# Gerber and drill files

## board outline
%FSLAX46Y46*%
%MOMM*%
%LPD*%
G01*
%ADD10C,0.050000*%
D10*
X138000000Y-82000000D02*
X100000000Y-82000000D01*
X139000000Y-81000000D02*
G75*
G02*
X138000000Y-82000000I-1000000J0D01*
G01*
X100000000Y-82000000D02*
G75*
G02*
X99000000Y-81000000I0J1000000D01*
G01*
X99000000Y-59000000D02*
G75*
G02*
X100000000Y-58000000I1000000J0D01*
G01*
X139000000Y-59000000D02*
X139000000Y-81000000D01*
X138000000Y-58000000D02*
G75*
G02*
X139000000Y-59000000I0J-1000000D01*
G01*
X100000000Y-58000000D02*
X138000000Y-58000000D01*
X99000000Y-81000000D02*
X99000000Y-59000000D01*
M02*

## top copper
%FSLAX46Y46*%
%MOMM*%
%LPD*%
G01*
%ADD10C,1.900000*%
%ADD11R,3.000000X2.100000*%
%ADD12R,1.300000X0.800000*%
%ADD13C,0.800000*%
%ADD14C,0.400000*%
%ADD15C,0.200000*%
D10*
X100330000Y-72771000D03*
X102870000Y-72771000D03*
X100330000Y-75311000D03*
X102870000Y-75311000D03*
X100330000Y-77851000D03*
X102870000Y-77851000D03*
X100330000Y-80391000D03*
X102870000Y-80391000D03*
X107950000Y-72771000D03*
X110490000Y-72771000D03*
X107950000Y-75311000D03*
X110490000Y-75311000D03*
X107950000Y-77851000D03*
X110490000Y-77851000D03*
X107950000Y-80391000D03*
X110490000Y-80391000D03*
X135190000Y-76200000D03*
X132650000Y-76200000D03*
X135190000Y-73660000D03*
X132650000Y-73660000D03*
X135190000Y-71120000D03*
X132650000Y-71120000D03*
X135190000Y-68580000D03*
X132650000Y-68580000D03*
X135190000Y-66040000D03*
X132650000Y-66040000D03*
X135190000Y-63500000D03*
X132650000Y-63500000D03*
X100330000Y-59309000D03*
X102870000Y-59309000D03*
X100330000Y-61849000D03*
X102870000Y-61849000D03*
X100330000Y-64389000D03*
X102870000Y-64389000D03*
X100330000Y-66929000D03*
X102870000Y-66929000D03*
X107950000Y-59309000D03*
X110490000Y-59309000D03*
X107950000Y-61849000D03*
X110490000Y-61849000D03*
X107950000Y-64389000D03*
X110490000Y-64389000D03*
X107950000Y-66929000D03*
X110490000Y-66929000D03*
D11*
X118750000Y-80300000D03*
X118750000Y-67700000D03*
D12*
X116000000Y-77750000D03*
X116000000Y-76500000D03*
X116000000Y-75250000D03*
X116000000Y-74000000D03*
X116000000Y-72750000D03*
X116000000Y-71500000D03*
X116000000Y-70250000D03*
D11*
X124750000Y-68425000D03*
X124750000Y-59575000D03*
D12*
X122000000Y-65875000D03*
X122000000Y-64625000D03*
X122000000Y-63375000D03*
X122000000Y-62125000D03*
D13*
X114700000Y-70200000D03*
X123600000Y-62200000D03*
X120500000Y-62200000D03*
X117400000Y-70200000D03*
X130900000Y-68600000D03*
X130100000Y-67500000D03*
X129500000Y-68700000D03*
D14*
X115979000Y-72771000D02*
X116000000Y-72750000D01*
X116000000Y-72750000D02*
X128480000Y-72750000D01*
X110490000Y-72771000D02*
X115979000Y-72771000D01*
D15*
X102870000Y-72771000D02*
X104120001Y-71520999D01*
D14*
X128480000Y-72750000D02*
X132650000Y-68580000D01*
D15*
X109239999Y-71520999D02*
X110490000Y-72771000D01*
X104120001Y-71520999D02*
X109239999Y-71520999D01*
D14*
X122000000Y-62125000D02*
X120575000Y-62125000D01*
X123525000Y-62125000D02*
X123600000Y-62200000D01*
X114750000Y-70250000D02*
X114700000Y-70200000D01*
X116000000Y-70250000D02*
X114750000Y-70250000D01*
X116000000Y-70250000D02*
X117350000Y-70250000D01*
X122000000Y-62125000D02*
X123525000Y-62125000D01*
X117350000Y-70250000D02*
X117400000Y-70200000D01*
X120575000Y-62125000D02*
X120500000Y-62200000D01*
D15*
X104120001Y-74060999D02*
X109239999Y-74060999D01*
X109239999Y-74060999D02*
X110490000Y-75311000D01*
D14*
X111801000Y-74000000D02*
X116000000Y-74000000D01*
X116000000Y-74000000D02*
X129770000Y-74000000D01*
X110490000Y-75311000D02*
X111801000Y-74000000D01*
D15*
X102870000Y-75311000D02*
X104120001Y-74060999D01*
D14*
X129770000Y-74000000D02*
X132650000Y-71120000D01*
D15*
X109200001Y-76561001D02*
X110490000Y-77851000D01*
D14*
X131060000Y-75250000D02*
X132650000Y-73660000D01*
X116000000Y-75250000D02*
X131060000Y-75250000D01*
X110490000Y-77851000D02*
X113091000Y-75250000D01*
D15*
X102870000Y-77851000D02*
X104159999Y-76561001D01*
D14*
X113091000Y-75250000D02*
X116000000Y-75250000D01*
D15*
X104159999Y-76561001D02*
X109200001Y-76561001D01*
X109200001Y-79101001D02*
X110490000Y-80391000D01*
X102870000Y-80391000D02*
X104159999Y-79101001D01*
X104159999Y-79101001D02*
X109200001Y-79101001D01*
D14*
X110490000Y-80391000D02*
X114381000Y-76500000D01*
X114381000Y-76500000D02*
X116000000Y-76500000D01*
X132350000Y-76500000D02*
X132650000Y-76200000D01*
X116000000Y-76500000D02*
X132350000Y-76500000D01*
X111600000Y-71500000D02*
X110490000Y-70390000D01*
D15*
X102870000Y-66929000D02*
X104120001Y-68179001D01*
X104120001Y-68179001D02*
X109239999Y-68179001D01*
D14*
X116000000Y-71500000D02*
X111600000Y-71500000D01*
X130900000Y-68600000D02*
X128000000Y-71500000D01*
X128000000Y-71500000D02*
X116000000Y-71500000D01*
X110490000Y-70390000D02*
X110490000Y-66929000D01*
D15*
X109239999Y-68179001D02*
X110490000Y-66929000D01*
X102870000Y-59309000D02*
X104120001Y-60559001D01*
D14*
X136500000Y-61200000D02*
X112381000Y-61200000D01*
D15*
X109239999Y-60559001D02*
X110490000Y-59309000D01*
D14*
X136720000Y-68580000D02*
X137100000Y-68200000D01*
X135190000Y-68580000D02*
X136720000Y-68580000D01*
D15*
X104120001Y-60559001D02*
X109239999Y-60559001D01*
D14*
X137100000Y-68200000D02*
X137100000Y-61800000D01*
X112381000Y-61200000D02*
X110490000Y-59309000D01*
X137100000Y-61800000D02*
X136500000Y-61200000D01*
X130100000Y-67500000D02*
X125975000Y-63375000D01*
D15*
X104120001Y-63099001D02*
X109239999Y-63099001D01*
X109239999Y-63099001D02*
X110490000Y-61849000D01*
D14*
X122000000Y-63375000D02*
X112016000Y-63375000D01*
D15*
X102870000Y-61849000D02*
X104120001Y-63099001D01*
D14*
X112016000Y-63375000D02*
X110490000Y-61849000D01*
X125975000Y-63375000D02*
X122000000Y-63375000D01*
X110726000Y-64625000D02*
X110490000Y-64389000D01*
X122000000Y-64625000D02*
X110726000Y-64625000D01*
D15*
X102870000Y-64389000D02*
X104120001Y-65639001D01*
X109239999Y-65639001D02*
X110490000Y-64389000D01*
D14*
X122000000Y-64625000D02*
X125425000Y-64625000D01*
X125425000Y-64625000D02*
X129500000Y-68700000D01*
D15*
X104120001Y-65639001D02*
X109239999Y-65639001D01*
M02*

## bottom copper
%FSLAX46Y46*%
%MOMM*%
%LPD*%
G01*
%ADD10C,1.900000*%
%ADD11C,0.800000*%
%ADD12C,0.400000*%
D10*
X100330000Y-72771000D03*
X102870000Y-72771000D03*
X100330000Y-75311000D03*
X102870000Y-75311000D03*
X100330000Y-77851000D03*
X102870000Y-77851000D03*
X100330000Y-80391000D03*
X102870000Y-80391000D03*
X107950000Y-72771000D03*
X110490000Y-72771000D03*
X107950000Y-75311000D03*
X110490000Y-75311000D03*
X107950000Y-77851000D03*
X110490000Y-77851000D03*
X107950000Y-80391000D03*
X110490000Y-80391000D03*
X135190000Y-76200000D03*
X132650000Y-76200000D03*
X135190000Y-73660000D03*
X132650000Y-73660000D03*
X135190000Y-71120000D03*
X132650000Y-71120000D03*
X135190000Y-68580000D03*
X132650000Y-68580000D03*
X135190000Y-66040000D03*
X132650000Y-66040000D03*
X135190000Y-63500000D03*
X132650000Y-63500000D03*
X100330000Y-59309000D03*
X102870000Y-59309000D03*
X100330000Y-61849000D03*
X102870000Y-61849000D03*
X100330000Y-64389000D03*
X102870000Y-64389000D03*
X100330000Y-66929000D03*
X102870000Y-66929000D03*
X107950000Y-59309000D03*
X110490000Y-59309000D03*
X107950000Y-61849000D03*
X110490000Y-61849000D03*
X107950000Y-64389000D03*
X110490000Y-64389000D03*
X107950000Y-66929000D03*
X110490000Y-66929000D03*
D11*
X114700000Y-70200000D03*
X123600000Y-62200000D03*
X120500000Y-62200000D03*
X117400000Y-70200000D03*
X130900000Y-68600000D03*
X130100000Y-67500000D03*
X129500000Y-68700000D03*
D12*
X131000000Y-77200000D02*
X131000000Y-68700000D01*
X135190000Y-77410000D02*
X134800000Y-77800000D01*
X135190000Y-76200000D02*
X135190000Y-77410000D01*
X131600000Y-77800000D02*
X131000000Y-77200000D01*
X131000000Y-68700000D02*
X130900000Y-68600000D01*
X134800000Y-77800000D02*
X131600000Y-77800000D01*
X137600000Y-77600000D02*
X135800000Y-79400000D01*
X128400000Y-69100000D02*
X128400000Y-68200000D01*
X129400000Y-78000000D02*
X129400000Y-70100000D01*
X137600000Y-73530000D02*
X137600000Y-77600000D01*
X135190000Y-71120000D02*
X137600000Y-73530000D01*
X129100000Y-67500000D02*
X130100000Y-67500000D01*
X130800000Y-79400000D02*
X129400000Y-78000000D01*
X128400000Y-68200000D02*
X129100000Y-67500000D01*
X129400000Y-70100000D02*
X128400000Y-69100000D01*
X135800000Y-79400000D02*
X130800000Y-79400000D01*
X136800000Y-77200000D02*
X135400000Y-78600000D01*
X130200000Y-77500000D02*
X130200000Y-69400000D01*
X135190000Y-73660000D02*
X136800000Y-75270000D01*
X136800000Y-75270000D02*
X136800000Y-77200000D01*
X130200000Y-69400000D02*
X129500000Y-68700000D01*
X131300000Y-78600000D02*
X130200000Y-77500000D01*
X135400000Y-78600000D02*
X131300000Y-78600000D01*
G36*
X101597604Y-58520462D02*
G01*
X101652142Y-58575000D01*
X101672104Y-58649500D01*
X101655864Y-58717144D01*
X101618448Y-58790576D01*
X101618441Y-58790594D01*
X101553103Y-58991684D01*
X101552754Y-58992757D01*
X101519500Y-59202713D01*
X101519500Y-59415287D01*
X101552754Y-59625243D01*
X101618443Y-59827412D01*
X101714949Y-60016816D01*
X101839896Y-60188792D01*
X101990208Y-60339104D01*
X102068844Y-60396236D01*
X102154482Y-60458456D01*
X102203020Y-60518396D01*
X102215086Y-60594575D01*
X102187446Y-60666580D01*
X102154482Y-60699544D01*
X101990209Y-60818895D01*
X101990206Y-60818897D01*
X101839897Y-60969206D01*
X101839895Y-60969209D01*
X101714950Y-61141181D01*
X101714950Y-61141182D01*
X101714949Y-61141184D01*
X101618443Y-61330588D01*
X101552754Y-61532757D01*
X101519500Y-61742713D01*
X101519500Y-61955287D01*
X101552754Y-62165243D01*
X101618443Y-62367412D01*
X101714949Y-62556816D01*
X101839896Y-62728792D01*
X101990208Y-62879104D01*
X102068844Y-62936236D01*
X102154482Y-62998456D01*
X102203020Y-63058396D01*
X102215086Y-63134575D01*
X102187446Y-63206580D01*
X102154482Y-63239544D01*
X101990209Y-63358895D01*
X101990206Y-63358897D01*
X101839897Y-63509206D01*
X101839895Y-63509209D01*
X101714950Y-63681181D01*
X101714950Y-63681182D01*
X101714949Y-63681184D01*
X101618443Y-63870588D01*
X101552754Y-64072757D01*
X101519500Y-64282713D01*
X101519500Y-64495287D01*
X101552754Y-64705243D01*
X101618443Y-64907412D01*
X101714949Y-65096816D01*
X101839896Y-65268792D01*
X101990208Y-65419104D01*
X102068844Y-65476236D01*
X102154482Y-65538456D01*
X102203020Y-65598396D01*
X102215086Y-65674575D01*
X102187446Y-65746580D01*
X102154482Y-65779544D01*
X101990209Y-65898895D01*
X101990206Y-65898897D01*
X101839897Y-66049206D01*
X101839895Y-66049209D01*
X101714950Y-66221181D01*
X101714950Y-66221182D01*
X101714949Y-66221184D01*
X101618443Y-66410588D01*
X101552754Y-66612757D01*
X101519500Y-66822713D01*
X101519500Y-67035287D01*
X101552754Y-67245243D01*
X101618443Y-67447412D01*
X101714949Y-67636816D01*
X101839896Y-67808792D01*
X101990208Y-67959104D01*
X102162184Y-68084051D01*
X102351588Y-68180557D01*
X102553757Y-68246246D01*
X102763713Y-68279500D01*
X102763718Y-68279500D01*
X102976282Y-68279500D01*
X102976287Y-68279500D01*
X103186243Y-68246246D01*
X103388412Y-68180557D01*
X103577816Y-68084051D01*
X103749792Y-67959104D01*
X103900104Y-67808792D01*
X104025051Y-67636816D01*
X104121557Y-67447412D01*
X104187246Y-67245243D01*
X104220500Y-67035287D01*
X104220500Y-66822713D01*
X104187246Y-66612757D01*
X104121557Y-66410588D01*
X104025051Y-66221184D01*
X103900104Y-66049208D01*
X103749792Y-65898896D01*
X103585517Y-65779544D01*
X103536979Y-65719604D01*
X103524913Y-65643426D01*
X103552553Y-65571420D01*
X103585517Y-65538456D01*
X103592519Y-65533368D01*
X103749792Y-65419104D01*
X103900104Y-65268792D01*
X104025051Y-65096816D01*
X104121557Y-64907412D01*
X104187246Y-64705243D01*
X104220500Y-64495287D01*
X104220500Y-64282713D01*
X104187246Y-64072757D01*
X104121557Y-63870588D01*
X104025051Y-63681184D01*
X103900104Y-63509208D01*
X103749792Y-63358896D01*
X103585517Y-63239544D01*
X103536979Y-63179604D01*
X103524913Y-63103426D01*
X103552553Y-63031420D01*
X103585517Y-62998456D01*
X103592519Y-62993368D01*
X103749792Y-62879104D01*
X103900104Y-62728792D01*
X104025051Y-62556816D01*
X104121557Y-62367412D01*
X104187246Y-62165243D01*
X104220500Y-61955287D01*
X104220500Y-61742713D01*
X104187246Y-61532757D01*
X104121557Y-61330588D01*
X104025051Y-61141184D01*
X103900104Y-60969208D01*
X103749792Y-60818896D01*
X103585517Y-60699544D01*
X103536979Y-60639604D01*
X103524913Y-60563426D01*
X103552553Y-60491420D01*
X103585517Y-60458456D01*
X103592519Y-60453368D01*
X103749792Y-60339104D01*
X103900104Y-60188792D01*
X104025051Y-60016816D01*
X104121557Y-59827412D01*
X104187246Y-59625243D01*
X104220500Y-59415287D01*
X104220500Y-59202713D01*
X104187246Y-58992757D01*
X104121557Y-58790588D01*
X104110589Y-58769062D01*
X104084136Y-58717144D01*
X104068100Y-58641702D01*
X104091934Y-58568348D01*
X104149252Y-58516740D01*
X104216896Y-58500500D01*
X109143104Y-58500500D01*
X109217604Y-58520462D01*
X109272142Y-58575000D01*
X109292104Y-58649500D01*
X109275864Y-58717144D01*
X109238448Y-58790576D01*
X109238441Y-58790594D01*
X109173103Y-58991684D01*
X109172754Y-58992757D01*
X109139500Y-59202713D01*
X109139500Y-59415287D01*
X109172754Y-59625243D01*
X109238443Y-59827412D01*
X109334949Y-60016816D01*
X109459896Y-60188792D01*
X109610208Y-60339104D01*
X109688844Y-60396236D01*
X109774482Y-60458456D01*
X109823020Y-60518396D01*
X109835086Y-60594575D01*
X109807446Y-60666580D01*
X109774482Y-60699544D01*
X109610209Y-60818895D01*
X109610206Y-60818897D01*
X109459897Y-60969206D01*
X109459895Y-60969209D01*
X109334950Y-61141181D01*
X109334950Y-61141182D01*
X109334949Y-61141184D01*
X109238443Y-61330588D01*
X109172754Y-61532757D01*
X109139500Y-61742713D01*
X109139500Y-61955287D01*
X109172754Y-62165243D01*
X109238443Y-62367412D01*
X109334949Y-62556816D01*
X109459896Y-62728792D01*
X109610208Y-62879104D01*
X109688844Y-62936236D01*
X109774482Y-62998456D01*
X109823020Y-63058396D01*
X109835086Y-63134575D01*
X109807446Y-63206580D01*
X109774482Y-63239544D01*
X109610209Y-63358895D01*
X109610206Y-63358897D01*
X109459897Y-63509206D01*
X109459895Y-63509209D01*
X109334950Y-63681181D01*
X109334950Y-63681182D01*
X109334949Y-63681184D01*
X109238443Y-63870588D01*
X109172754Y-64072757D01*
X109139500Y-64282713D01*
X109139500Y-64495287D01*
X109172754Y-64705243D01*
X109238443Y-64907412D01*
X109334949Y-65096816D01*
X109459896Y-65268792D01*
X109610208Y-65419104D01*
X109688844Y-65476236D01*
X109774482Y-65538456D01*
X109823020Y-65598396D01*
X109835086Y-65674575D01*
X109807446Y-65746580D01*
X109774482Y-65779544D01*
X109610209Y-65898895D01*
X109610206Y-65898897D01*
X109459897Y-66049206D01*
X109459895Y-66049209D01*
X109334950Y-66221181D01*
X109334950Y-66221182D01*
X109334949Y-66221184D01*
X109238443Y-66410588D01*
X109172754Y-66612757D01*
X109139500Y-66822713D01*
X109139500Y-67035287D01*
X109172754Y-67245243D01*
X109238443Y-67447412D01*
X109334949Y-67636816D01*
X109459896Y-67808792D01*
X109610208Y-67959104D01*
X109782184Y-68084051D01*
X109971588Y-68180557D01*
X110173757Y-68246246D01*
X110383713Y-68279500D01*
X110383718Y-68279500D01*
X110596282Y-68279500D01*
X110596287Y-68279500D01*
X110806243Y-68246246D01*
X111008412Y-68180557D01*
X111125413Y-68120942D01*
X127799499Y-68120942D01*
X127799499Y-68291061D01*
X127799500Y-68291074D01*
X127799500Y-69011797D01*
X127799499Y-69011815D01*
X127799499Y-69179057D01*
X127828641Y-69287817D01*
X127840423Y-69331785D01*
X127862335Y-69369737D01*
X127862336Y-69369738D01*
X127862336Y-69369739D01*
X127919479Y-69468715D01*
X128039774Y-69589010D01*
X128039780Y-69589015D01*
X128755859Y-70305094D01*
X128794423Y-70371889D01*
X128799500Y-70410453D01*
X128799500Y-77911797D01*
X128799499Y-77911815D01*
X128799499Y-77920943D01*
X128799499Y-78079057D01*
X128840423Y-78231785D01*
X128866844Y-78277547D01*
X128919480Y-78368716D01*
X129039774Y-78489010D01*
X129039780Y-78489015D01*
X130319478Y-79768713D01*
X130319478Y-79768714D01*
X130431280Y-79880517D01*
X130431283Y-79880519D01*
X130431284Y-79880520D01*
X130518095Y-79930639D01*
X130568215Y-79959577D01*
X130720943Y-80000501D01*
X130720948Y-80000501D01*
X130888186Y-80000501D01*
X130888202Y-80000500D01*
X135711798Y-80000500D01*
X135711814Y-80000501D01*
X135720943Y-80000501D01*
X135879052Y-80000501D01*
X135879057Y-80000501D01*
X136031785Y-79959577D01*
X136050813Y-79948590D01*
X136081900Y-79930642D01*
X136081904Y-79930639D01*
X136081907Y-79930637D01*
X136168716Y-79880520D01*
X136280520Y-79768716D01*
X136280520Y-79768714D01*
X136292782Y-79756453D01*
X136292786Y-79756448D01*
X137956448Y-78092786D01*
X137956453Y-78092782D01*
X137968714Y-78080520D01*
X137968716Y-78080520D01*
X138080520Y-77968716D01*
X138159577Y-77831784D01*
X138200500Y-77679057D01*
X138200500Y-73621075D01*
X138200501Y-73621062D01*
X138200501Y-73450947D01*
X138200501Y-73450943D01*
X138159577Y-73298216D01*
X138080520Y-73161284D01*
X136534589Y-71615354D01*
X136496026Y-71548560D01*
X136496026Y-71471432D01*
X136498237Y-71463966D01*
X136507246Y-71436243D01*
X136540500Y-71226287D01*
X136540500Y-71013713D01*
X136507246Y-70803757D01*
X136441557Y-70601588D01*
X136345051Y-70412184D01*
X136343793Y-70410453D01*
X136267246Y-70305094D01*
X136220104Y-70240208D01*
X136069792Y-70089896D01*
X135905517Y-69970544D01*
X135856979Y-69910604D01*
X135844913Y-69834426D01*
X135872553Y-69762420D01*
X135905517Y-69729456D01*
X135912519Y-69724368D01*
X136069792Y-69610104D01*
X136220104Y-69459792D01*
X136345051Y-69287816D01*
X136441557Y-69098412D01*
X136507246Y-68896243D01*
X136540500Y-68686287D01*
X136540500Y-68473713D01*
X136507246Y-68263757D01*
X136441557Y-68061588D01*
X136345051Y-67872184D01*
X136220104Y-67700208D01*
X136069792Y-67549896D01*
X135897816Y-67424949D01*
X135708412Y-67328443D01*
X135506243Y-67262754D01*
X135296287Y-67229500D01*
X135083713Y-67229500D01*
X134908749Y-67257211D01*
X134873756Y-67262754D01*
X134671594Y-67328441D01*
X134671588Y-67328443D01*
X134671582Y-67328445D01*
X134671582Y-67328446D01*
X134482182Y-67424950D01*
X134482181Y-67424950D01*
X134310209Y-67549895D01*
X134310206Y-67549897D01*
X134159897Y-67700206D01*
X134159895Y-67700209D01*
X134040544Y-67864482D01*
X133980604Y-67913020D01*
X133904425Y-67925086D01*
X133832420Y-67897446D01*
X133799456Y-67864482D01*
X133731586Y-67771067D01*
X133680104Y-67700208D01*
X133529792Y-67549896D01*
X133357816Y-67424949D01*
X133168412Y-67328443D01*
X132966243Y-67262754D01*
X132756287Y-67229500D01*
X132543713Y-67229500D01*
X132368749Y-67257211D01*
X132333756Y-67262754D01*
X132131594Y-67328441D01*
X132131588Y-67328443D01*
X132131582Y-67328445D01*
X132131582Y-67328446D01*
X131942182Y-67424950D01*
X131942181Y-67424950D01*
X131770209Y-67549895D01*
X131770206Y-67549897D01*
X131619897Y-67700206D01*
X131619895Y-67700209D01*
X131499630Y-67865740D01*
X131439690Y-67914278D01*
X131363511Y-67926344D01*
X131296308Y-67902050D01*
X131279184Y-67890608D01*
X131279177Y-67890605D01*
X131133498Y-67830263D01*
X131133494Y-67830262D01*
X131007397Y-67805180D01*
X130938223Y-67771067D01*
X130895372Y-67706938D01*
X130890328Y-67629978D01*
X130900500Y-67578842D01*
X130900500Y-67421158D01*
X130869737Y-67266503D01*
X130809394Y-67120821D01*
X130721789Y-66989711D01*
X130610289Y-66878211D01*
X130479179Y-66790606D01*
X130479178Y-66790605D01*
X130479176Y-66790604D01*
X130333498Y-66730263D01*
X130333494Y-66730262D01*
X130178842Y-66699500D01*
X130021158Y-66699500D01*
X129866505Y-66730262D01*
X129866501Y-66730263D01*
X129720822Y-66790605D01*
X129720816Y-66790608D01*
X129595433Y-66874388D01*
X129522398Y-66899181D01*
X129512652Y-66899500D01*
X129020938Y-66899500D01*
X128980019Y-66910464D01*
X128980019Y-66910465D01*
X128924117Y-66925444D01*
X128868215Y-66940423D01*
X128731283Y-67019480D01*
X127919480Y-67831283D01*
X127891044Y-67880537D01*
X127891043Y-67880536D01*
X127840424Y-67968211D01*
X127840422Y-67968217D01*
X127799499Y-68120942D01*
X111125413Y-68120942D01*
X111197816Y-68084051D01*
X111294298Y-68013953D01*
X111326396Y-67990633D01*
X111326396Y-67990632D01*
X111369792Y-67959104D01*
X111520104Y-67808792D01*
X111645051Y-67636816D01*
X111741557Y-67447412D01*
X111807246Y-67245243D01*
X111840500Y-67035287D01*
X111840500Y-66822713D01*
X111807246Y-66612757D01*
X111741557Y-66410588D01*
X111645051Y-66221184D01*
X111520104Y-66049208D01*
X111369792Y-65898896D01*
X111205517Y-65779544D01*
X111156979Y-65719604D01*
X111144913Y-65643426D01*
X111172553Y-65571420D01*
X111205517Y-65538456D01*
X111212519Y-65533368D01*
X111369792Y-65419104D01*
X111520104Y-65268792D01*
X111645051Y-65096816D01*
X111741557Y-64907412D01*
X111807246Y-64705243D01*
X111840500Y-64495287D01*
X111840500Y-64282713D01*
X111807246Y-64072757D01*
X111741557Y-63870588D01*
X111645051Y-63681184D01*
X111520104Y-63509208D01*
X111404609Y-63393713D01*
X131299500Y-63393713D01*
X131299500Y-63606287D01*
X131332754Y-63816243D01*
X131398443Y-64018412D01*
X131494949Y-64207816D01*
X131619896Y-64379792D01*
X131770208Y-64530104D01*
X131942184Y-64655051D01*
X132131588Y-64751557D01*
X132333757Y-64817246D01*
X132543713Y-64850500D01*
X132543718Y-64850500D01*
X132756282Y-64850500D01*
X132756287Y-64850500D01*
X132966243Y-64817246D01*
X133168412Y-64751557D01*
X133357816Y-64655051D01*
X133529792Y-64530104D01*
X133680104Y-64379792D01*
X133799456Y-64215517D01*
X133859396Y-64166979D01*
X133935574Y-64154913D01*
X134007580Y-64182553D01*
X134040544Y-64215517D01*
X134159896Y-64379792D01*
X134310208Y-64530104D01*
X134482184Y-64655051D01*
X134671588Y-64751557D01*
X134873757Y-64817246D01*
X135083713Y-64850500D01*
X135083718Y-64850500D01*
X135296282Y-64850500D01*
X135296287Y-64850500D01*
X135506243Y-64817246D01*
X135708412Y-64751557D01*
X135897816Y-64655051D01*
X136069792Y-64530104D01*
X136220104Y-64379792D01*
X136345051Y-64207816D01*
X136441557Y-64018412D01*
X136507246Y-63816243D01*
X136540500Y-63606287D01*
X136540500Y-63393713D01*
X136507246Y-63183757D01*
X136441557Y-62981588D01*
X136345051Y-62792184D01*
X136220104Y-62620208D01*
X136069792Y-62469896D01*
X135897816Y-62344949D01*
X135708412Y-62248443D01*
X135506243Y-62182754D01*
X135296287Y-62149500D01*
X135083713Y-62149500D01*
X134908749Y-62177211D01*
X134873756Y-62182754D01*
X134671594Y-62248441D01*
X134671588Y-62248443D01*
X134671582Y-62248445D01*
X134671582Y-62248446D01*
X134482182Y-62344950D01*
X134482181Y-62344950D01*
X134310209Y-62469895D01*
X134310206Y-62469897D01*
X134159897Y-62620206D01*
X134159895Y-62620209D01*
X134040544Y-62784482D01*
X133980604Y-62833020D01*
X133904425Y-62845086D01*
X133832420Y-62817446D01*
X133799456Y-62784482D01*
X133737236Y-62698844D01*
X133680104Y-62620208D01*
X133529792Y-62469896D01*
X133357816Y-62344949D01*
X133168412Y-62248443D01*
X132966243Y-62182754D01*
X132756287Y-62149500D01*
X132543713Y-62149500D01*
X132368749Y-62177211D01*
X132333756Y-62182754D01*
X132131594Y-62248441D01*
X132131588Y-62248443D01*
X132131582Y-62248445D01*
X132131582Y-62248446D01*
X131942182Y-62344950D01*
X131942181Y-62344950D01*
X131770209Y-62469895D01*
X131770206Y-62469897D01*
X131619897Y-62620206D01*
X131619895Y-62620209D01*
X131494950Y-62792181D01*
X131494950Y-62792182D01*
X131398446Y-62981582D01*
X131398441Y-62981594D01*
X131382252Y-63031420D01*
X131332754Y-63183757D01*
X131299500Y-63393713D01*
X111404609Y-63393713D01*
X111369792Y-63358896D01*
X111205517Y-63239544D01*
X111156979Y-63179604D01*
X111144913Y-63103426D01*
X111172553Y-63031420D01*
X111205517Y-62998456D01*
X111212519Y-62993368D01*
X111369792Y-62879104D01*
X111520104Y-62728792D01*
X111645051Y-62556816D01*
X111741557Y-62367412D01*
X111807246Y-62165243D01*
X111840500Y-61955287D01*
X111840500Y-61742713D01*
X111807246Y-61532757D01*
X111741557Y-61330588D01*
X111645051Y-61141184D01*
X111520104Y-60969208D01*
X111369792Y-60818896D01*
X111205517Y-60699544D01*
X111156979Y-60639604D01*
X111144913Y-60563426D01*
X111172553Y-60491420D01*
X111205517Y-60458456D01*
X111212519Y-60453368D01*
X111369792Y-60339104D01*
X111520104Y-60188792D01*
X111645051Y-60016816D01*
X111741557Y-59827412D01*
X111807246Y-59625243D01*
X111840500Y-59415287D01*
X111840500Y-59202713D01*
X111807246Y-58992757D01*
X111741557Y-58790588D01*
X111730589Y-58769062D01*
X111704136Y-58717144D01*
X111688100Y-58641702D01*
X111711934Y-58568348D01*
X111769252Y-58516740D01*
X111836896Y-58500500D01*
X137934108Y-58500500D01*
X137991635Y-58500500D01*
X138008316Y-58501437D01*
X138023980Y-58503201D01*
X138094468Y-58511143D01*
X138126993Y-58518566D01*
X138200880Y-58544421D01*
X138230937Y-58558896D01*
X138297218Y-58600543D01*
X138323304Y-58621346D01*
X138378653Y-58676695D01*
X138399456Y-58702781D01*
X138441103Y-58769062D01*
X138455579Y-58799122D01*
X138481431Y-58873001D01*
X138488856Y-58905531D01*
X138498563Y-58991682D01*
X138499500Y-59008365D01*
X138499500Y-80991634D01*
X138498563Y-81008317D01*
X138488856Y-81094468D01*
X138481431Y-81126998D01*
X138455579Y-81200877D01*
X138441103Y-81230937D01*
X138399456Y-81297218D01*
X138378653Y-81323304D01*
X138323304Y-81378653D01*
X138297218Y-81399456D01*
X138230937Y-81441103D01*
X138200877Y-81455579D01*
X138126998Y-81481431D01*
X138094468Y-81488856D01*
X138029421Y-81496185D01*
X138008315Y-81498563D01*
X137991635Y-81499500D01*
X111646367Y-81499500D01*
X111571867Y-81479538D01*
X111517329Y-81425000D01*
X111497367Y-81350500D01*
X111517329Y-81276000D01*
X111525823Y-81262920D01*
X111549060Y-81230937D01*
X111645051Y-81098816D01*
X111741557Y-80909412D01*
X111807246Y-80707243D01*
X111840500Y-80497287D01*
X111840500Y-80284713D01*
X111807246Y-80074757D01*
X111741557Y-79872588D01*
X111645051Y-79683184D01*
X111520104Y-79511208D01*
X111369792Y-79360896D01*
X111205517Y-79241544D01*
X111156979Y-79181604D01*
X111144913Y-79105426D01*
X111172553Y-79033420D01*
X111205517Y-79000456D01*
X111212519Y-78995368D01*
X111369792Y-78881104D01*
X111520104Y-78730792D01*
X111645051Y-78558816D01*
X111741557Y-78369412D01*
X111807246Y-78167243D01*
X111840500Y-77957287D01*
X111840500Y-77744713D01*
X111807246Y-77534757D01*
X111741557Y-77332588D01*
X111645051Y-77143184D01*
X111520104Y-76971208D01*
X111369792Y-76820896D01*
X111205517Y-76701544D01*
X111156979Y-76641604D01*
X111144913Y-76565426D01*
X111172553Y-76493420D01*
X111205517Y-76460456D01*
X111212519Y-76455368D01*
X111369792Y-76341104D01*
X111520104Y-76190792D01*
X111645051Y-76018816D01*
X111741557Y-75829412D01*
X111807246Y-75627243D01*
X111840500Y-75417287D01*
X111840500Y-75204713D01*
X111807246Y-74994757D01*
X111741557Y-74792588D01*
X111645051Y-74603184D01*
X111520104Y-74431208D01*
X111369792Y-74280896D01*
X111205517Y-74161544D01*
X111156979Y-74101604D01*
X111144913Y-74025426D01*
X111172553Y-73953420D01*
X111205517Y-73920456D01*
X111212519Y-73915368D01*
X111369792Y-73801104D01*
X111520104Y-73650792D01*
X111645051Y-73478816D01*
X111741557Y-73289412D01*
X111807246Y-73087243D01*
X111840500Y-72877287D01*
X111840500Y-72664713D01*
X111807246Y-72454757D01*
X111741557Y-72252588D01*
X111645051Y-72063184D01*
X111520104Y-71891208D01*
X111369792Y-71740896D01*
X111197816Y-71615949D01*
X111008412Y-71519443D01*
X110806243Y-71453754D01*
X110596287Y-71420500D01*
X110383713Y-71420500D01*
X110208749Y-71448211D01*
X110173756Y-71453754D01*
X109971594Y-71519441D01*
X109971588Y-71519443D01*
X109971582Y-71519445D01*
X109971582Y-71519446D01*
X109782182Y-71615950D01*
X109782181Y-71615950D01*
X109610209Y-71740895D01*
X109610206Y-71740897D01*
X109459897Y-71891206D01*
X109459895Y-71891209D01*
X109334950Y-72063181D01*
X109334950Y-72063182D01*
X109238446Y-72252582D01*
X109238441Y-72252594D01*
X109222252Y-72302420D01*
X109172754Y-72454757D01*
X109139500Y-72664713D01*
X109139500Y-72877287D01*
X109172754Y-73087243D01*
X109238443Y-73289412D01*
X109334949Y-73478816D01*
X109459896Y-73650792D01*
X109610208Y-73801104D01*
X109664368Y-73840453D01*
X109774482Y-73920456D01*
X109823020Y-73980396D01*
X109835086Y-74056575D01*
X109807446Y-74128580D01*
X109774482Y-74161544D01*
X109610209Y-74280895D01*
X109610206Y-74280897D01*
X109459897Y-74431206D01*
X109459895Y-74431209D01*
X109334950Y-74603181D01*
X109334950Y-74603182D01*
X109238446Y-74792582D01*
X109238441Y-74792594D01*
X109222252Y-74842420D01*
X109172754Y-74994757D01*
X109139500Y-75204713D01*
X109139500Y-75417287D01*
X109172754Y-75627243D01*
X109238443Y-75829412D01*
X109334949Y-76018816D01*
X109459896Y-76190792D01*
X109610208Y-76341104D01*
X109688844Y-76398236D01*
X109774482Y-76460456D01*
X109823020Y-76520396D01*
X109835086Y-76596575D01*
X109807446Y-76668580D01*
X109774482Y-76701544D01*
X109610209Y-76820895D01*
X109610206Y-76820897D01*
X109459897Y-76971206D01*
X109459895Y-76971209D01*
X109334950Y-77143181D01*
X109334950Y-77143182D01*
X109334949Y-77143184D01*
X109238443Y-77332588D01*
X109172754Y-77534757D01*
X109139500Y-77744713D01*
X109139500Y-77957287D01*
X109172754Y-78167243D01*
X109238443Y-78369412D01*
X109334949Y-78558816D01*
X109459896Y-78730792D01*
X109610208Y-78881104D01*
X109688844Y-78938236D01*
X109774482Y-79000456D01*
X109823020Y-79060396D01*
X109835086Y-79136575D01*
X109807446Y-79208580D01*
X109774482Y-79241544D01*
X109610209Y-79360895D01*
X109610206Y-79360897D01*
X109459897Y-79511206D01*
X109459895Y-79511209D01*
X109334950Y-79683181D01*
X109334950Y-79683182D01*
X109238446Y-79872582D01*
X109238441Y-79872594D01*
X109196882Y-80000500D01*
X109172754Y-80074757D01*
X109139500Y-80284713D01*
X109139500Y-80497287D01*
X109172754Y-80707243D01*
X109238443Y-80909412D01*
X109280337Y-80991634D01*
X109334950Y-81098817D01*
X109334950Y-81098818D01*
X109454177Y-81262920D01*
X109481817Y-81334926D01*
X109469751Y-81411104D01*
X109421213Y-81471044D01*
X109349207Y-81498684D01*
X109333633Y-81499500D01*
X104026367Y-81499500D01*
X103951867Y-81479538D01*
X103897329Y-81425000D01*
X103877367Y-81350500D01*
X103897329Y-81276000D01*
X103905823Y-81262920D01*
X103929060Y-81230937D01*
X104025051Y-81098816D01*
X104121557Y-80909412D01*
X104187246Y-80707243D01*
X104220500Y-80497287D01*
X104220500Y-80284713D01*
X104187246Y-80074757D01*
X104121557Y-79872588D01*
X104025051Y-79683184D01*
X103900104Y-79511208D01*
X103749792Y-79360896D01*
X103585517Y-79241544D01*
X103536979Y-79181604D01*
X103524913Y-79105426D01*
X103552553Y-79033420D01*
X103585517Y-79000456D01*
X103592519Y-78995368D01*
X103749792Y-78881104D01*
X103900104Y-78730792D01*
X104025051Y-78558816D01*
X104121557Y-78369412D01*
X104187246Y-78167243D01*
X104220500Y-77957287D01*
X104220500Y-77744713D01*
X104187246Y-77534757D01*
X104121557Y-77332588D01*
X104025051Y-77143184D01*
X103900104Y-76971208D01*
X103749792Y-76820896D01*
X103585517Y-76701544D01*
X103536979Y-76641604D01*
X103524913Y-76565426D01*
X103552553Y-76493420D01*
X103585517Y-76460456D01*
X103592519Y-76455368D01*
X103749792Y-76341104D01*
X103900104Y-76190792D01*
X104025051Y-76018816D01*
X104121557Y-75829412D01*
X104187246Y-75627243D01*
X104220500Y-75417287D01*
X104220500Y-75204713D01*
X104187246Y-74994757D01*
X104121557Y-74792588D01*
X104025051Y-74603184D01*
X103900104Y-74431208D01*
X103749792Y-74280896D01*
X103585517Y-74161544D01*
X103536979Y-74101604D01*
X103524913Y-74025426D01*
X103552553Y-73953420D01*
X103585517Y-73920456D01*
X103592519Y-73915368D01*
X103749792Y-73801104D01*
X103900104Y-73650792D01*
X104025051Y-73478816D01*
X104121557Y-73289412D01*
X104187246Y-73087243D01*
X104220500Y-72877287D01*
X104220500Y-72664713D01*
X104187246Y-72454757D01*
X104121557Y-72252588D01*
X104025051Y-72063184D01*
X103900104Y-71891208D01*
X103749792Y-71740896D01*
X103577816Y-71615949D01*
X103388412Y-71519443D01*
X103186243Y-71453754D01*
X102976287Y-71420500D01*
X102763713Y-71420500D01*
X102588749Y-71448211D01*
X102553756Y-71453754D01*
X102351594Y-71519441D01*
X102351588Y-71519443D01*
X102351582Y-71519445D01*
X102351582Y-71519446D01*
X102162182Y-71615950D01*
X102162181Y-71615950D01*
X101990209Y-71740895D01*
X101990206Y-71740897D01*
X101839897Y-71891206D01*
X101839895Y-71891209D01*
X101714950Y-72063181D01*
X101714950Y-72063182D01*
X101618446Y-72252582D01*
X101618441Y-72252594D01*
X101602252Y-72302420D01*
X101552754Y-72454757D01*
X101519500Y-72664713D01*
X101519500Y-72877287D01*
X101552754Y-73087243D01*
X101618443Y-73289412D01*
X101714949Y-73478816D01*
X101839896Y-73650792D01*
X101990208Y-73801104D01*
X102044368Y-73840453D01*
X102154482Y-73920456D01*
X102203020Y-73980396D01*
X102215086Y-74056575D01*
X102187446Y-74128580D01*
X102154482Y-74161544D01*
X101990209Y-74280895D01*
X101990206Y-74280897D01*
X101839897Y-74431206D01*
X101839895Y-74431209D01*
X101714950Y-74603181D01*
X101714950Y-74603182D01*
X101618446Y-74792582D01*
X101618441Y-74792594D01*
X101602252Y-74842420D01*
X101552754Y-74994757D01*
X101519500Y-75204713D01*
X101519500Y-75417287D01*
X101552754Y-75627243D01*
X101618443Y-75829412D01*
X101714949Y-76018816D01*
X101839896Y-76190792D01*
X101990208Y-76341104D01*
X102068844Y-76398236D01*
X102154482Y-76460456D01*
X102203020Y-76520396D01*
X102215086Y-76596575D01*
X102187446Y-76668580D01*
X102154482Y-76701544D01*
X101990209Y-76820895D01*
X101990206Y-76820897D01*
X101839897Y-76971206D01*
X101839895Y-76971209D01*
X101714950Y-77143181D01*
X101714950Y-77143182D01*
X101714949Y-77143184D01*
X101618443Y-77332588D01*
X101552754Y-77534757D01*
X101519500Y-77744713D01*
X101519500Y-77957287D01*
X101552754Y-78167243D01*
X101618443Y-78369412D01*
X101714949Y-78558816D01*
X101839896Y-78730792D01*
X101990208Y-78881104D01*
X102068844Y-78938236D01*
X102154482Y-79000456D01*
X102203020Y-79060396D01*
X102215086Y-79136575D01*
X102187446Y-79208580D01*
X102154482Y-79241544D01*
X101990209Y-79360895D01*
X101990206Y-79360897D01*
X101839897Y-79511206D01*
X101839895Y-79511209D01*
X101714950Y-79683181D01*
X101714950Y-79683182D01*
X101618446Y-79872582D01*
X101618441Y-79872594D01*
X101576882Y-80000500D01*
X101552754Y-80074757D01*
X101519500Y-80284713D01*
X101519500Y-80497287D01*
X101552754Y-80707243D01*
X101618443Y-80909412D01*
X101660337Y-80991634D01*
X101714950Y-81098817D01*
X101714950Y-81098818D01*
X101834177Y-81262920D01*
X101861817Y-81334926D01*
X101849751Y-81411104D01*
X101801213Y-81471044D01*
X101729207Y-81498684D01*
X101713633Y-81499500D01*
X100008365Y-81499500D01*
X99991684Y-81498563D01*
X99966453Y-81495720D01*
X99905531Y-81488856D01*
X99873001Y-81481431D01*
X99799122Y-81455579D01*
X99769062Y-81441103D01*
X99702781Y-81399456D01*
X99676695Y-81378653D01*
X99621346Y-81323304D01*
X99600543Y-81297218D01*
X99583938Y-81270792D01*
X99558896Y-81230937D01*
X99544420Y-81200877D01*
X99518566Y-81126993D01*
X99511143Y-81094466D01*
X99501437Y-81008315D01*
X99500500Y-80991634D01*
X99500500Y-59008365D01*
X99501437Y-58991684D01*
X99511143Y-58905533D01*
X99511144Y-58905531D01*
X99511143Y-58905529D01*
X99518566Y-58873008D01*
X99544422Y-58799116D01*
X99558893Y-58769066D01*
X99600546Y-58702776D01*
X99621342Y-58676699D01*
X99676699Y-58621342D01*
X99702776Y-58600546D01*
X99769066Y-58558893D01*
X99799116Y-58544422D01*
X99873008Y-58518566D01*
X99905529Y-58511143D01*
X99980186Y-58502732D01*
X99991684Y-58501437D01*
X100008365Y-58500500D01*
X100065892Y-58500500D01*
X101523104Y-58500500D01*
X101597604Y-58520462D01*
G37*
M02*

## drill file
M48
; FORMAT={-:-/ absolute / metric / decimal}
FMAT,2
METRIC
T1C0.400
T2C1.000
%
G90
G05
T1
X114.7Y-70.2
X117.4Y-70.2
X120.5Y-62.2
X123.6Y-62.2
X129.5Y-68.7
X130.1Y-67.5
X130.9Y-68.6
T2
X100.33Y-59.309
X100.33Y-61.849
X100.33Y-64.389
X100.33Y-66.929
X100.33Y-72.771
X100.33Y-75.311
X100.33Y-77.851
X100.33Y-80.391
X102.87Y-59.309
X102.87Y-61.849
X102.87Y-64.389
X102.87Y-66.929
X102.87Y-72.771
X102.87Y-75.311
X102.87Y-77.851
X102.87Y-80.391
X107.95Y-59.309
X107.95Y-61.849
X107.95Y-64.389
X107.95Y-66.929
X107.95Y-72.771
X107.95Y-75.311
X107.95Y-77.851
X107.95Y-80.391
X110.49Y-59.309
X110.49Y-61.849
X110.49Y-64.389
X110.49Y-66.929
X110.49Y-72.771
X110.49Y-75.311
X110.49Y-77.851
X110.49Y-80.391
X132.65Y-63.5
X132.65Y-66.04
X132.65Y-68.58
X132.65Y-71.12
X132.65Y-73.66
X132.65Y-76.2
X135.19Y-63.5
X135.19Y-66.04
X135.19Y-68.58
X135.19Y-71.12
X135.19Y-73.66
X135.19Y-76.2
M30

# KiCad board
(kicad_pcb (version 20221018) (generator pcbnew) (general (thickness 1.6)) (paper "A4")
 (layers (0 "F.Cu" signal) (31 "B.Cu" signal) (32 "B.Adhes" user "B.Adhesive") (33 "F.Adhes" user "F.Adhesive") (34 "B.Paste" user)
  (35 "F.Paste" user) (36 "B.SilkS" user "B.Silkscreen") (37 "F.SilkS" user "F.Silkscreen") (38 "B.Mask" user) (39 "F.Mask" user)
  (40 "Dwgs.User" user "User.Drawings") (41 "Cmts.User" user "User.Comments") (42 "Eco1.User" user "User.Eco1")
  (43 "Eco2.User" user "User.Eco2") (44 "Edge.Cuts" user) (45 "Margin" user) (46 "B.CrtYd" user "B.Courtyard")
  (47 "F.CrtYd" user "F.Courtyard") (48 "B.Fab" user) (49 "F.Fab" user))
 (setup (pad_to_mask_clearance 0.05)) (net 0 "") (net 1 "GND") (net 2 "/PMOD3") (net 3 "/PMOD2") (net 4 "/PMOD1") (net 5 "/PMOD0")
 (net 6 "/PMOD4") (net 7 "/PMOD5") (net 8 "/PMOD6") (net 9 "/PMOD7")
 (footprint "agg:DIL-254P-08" (layer "F.Cu") (at 101.6 76.581 -90)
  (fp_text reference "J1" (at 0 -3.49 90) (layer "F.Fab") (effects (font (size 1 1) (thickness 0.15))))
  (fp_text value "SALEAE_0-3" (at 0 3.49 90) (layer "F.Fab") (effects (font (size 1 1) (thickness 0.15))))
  (pad "1" thru_hole circle (at -3.81 1.27 270) (size 1.9 1.9) (drill 1) (layers "*.Cu" "*.Mask" "F.SilkS") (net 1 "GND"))
  (pad "2" thru_hole circle (at -3.81 -1.27 270) (size 1.9 1.9) (drill 1) (layers "*.Cu" "*.Mask" "F.SilkS") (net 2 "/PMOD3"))
  (pad "3" thru_hole circle (at -1.27 1.27 270) (size 1.9 1.9) (drill 1) (layers "*.Cu" "*.Mask" "F.SilkS") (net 1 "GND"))
  (pad "4" thru_hole circle (at -1.27 -1.27 270) (size 1.9 1.9) (drill 1) (layers "*.Cu" "*.Mask" "F.SilkS") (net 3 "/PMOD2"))
  (pad "5" thru_hole circle (at 1.27 1.27 270) (size 1.9 1.9) (drill 1) (layers "*.Cu" "*.Mask" "F.SilkS") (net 1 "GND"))
  (pad "6" thru_hole circle (at 1.27 -1.27 270) (size 1.9 1.9) (drill 1) (layers "*.Cu" "*.Mask" "F.SilkS") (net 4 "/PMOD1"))
  (pad "7" thru_hole circle (at 3.81 1.27 270) (size 1.9 1.9) (drill 1) (layers "*.Cu" "*.Mask" "F.SilkS") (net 1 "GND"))
  (pad "8" thru_hole circle (at 3.81 -1.27 270) (size 1.9 1.9) (drill 1) (layers "*.Cu" "*.Mask" "F.SilkS") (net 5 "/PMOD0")))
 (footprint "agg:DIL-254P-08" (layer "F.Cu") (at 109.22 76.581 -90)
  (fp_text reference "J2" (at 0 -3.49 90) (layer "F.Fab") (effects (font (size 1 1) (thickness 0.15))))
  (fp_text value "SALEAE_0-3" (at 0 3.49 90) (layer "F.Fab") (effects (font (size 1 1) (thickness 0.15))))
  (pad "1" thru_hole circle (at -3.81 1.27 270) (size 1.9 1.9) (drill 1) (layers "*.Cu" "*.Mask" "F.SilkS") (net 1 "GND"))
  (pad "2" thru_hole circle (at -3.81 -1.27 270) (size 1.9 1.9) (drill 1) (layers "*.Cu" "*.Mask" "F.SilkS") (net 2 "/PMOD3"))
  (pad "3" thru_hole circle (at -1.27 1.27 270) (size 1.9 1.9) (drill 1) (layers "*.Cu" "*.Mask" "F.SilkS") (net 1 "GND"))
  (pad "4" thru_hole circle (at -1.27 -1.27 270) (size 1.9 1.9) (drill 1) (layers "*.Cu" "*.Mask" "F.SilkS") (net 3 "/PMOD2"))
  (pad "5" thru_hole circle (at 1.27 1.27 270) (size 1.9 1.9) (drill 1) (layers "*.Cu" "*.Mask" "F.SilkS") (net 1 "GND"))
  (pad "6" thru_hole circle (at 1.27 -1.27 270) (size 1.9 1.9) (drill 1) (layers "*.Cu" "*.Mask" "F.SilkS") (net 4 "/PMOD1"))
  (pad "7" thru_hole circle (at 3.81 1.27 270) (size 1.9 1.9) (drill 1) (layers "*.Cu" "*.Mask" "F.SilkS") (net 1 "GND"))
  (pad "8" thru_hole circle (at 3.81 -1.27 270) (size 1.9 1.9) (drill 1) (layers "*.Cu" "*.Mask" "F.SilkS") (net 5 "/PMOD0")))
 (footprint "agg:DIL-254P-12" (layer "F.Cu") (at 133.92 69.85 90)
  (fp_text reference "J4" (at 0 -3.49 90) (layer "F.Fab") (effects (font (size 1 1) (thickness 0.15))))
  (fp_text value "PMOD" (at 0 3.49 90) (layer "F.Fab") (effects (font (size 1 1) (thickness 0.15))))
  (pad "1" thru_hole circle (at -6.35 1.27 90) (size 1.9 1.9) (drill 1) (layers "*.Cu" "*.Mask" "F.SilkS") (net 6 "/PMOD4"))
  (pad "2" thru_hole circle (at -6.35 -1.27 90) (size 1.9 1.9) (drill 1) (layers "*.Cu" "*.Mask" "F.SilkS") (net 5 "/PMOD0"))
  (pad "3" thru_hole circle (at -3.81 1.27 90) (size 1.9 1.9) (drill 1) (layers "*.Cu" "*.Mask" "F.SilkS") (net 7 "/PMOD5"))
  (pad "4" thru_hole circle (at -3.81 -1.27 90) (size 1.9 1.9) (drill 1) (layers "*.Cu" "*.Mask" "F.SilkS") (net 4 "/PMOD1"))
  (pad "5" thru_hole circle (at -1.27 1.27 90) (size 1.9 1.9) (drill 1) (layers "*.Cu" "*.Mask" "F.SilkS") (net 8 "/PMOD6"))
  (pad "6" thru_hole circle (at -1.27 -1.27 90) (size 1.9 1.9) (drill 1) (layers "*.Cu" "*.Mask" "F.SilkS") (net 3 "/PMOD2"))
  (pad "7" thru_hole circle (at 1.27 1.27 90) (size 1.9 1.9) (drill 1) (layers "*.Cu" "*.Mask" "F.SilkS") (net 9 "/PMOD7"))
  (pad "8" thru_hole circle (at 1.27 -1.27 90) (size 1.9 1.9) (drill 1) (layers "*.Cu" "*.Mask" "F.SilkS") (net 2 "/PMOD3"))
  (pad "9" thru_hole circle (at 3.81 1.27 90) (size 1.9 1.9) (drill 1) (layers "*.Cu" "*.Mask" "F.SilkS") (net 1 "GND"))
  (pad "10" thru_hole circle (at 3.81 -1.27 90) (size 1.9 1.9) (drill 1) (layers "*.Cu" "*.Mask" "F.SilkS") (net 1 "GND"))
  (pad "11" thru_hole circle (at 6.35 1.27 90) (size 1.9 1.9) (drill 1) (layers "*.Cu" "*.Mask" "F.SilkS"))
  (pad "12" thru_hole circle (at 6.35 -1.27 90) (size 1.9 1.9) (drill 1) (layers "*.Cu" "*.Mask" "F.SilkS")))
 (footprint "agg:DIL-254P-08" (layer "F.Cu") (at 101.6 63.119 -90)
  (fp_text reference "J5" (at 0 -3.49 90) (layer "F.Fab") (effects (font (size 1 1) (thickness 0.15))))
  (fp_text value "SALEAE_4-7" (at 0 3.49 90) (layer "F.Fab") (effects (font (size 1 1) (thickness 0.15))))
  (pad "1" thru_hole circle (at -3.81 1.27 270) (size 1.9 1.9) (drill 1) (layers "*.Cu" "*.Mask" "F.SilkS") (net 1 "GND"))
  (pad "2" thru_hole circle (at -3.81 -1.27 270) (size 1.9 1.9) (drill 1) (layers "*.Cu" "*.Mask" "F.SilkS") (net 9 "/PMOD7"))
  (pad "3" thru_hole circle (at -1.27 1.27 270) (size 1.9 1.9) (drill 1) (layers "*.Cu" "*.Mask" "F.SilkS") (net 1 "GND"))
  (pad "4" thru_hole circle (at -1.27 -1.27 270) (size 1.9 1.9) (drill 1) (layers "*.Cu" "*.Mask" "F.SilkS") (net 8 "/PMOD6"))
  (pad "5" thru_hole circle (at 1.27 1.27 270) (size 1.9 1.9) (drill 1) (layers "*.Cu" "*.Mask" "F.SilkS") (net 1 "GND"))
  (pad "6" thru_hole circle (at 1.27 -1.27 270) (size 1.9 1.9) (drill 1) (layers "*.Cu" "*.Mask" "F.SilkS") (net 7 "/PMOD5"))
  (pad "7" thru_hole circle (at 3.81 1.27 270) (size 1.9 1.9) (drill 1) (layers "*.Cu" "*.Mask" "F.SilkS") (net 1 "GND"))
  (pad "8" thru_hole circle (at 3.81 -1.27 270) (size 1.9 1.9) (drill 1) (layers "*.Cu" "*.Mask" "F.SilkS") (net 6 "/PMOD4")))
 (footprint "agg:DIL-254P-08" (layer "F.Cu") (at 109.22 63.119 -90)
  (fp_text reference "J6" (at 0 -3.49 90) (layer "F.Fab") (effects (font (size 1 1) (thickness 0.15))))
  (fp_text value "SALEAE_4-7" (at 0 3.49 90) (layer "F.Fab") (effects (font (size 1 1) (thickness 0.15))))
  (pad "1" thru_hole circle (at -3.81 1.27 270) (size 1.9 1.9) (drill 1) (layers "*.Cu" "*.Mask" "F.SilkS") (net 1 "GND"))
  (pad "2" thru_hole circle (at -3.81 -1.27 270) (size 1.9 1.9) (drill 1) (layers "*.Cu" "*.Mask" "F.SilkS") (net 9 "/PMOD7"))
  (pad "3" thru_hole circle (at -1.27 1.27 270) (size 1.9 1.9) (drill 1) (layers "*.Cu" "*.Mask" "F.SilkS") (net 1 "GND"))
  (pad "4" thru_hole circle (at -1.27 -1.27 270) (size 1.9 1.9) (drill 1) (layers "*.Cu" "*.Mask" "F.SilkS") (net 8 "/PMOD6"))
  (pad "5" thru_hole circle (at 1.27 1.27 270) (size 1.9 1.9) (drill 1) (layers "*.Cu" "*.Mask" "F.SilkS") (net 1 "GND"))
  (pad "6" thru_hole circle (at 1.27 -1.27 270) (size 1.9 1.9) (drill 1) (layers "*.Cu" "*.Mask" "F.SilkS") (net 7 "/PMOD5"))
  (pad "7" thru_hole circle (at 3.81 1.27 270) (size 1.9 1.9) (drill 1) (layers "*.Cu" "*.Mask" "F.SilkS") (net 1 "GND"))
  (pad "8" thru_hole circle (at 3.81 -1.27 270) (size 1.9 1.9) (drill 1) (layers "*.Cu" "*.Mask" "F.SilkS") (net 6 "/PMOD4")))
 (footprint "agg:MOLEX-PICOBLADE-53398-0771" (layer "F.Cu") (at 116 74 90)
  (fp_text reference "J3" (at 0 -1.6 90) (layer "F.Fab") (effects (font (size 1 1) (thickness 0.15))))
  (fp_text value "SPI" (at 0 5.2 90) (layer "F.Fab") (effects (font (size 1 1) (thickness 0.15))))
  (pad "" smd rect (at -6.3 2.75 90) (size 2.1 3) (layers "F.Cu" "F.Paste" "F.Mask"))
  (pad "" smd rect (at 6.3 2.75 90) (size 2.1 3) (layers "F.Cu" "F.Paste" "F.Mask"))
  (pad "1" smd rect (at -3.75 0 90) (size 0.8 1.3) (layers "F.Cu" "F.Paste" "F.Mask"))
  (pad "2" smd rect (at -2.5 0 90) (size 0.8 1.3) (layers "F.Cu" "F.Paste" "F.Mask") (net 5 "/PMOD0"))
  (pad "3" smd rect (at -1.25 0 90) (size 0.8 1.3) (layers "F.Cu" "F.Paste" "F.Mask") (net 4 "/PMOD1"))
  (pad "4" smd rect (at 0 0 90) (size 0.8 1.3) (layers "F.Cu" "F.Paste" "F.Mask") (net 3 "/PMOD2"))
  (pad "5" smd rect (at 1.25 0 90) (size 0.8 1.3) (layers "F.Cu" "F.Paste" "F.Mask") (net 2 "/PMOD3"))
  (pad "6" smd rect (at 2.5 0 90) (size 0.8 1.3) (layers "F.Cu" "F.Paste" "F.Mask") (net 6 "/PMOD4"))
  (pad "7" smd rect (at 3.75 0 90) (size 0.8 1.3) (layers "F.Cu" "F.Paste" "F.Mask") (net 1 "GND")))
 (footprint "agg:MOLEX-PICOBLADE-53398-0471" (layer "F.Cu") (at 122 64 90)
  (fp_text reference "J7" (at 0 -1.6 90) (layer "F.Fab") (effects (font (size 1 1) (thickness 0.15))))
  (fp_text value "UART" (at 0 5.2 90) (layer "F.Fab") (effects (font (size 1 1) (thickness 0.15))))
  (pad "" smd rect (at -4.425 2.75 90) (size 2.1 3) (layers "F.Cu" "F.Paste" "F.Mask"))
  (pad "" smd rect (at 4.425 2.75 90) (size 2.1 3) (layers "F.Cu" "F.Paste" "F.Mask"))
  (pad "1" smd rect (at -1.875 0 90) (size 0.8 1.3) (layers "F.Cu" "F.Paste" "F.Mask"))
  (pad "2" smd rect (at -0.625 0 90) (size 0.8 1.3) (layers "F.Cu" "F.Paste" "F.Mask") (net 7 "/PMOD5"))
  (pad "3" smd rect (at 0.625 0 90) (size 0.8 1.3) (layers "F.Cu" "F.Paste" "F.Mask") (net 8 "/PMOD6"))
  (pad "4" smd rect (at 1.875 0 90) (size 0.8 1.3) (layers "F.Cu" "F.Paste" "F.Mask") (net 1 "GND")))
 (gr_line (start 138 82) (end 100 82) (stroke (width 0.05) (type solid)) (layer "Edge.Cuts"))
 (gr_arc (start 139 81) (mid 138.707107 81.707107) (end 138 82) (stroke (width 0.05) (type solid)) (layer "Edge.Cuts"))
 (gr_arc (start 100 82) (mid 99.292893 81.707107) (end 99 81) (stroke (width 0.05) (type solid)) (layer "Edge.Cuts"))
 (gr_arc (start 99 59) (mid 99.292893 58.292893) (end 100 58) (stroke (width 0.05) (type solid)) (layer "Edge.Cuts"))
 (gr_line (start 139 59) (end 139 81) (stroke (width 0.05) (type solid)) (layer "Edge.Cuts"))
 (gr_arc (start 138 58) (mid 138.707107 58.292893) (end 139 59) (stroke (width 0.05) (type solid)) (layer "Edge.Cuts"))
 (gr_line (start 100 58) (end 138 58) (stroke (width 0.05) (type solid)) (layer "Edge.Cuts"))
 (gr_line (start 99 81) (end 99 59) (stroke (width 0.05) (type solid)) (layer "Edge.Cuts"))
 (segment (start 115.979 72.771) (end 116 72.75) (width 0.4) (layer "F.Cu") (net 2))
 (segment (start 116 72.75) (end 128.48 72.75) (width 0.4) (layer "F.Cu") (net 2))
 (segment (start 110.49 72.771) (end 115.979 72.771) (width 0.4) (layer "F.Cu") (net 2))
 (segment (start 102.87 72.771) (end 104.120001 71.520999) (width 0.2) (layer "F.Cu") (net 2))
 (segment (start 128.48 72.75) (end 132.65 68.58) (width 0.4) (layer "F.Cu") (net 2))
 (segment (start 109.239999 71.520999) (end 110.49 72.771) (width 0.2) (layer "F.Cu") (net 2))
 (segment (start 104.120001 71.520999) (end 109.239999 71.520999) (width 0.2) (layer "F.Cu") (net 2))
 (segment (start 122 62.125) (end 120.575 62.125) (width 0.4) (layer "F.Cu") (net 1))
 (segment (start 123.525 62.125) (end 123.6 62.2) (width 0.4) (layer "F.Cu") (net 1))
 (segment (start 114.75 70.25) (end 114.7 70.2) (width 0.4) (layer "F.Cu") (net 1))
 (segment (start 116 70.25) (end 114.75 70.25) (width 0.4) (layer "F.Cu") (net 1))
 (segment (start 116 70.25) (end 117.35 70.25) (width 0.4) (layer "F.Cu") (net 1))
 (segment (start 122 62.125) (end 123.525 62.125) (width 0.4) (layer "F.Cu") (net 1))
 (segment (start 117.35 70.25) (end 117.4 70.2) (width 0.4) (layer "F.Cu") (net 1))
 (segment (start 120.575 62.125) (end 120.5 62.2) (width 0.4) (layer "F.Cu") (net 1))
 (via (at 114.7 70.2) (size 0.8) (drill 0.4) (layers "F.Cu" "B.Cu") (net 1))
 (via (at 123.6 62.2) (size 0.8) (drill 0.4) (layers "F.Cu" "B.Cu") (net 1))
 (via (at 120.5 62.2) (size 0.8) (drill 0.4) (layers "F.Cu" "B.Cu") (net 1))
 (via (at 117.4 70.2) (size 0.8) (drill 0.4) (layers "F.Cu" "B.Cu") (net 1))
 (segment (start 104.120001 74.060999) (end 109.239999 74.060999) (width 0.2) (layer "F.Cu") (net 3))
 (segment (start 109.239999 74.060999) (end 110.49 75.311) (width 0.2) (layer "F.Cu") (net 3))
 (segment (start 111.801 74) (end 116 74) (width 0.4) (layer "F.Cu") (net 3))
 (segment (start 116 74) (end 129.77 74) (width 0.4) (layer "F.Cu") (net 3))
 (segment (start 110.49 75.311) (end 111.801 74) (width 0.4) (layer "F.Cu") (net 3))
 (segment (start 102.87 75.311) (end 104.120001 74.060999) (width 0.2) (layer "F.Cu") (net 3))
 (segment (start 129.77 74) (end 132.65 71.12) (width 0.4) (layer "F.Cu") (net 3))
 (segment (start 109.200001 76.561001) (end 110.49 77.851) (width 0.2) (layer "F.Cu") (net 4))
 (segment (start 131.06 75.25) (end 132.65 73.66) (width 0.4) (layer "F.Cu") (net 4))
 (segment (start 116 75.25) (end 131.06 75.25) (width 0.4) (layer "F.Cu") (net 4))
 (segment (start 110.49 77.851) (end 113.091 75.25) (width 0.4) (layer "F.Cu") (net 4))
 (segment (start 102.87 77.851) (end 104.159999 76.561001) (width 0.2) (layer "F.Cu") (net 4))
 (segment (start 113.091 75.25) (end 116 75.25) (width 0.4) (layer "F.Cu") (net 4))
 (segment (start 104.159999 76.561001) (end 109.200001 76.561001) (width 0.2) (layer "F.Cu") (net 4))
 (segment (start 109.200001 79.101001) (end 110.49 80.391) (width 0.2) (layer "F.Cu") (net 5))
 (segment (start 102.87 80.391) (end 104.159999 79.101001) (width 0.2) (layer "F.Cu") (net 5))
 (segment (start 104.159999 79.101001) (end 109.200001 79.101001) (width 0.2) (layer "F.Cu") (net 5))
 (segment (start 110.49 80.391) (end 114.381 76.5) (width 0.4) (layer "F.Cu") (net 5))
 (segment (start 114.381 76.5) (end 116 76.5) (width 0.4) (layer "F.Cu") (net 5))
 (segment (start 132.35 76.5) (end 132.65 76.2) (width 0.4) (layer "F.Cu") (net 5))
 (segment (start 116 76.5) (end 132.35 76.5) (width 0.4) (layer "F.Cu") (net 5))
 (segment (start 111.6 71.5) (end 110.49 70.39) (width 0.4) (layer "F.Cu") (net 6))
 (segment (start 102.87 66.929) (end 104.120001 68.179001) (width 0.2) (layer "F.Cu") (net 6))
 (segment (start 104.120001 68.179001) (end 109.239999 68.179001) (width 0.2) (layer "F.Cu") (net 6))
 (segment (start 116 71.5) (end 111.6 71.5) (width 0.4) (layer "F.Cu") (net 6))
 (segment (start 130.9 68.6) (end 128 71.5) (width 0.4) (layer "F.Cu") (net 6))
 (segment (start 128 71.5) (end 116 71.5) (width 0.4) (layer "F.Cu") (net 6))
 (segment (start 110.49 70.39) (end 110.49 66.929) (width 0.4) (layer "F.Cu") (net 6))
 (segment (start 109.239999 68.179001) (end 110.49 66.929) (width 0.2) (layer "F.Cu") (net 6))
 (via (at 130.9 68.6) (size 0.8) (drill 0.4) (layers "F.Cu" "B.Cu") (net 6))
 (segment (start 131 77.2) (end 131 68.7) (width 0.4) (layer "B.Cu") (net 6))
 (segment (start 135.19 77.41) (end 134.8 77.8) (width 0.4) (layer "B.Cu") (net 6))
 (segment (start 135.19 76.2) (end 135.19 77.41) (width 0.4) (layer "B.Cu") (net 6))
 (segment (start 131.6 77.8) (end 131 77.2) (width 0.4) (layer "B.Cu") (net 6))
 (segment (start 131 68.7) (end 130.9 68.6) (width 0.4) (layer "B.Cu") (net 6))
 (segment (start 134.8 77.8) (end 131.6 77.8) (width 0.4) (layer "B.Cu") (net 6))
 (segment (start 102.87 59.309) (end 104.120001 60.559001) (width 0.2) (layer "F.Cu") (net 9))
 (segment (start 136.5 61.2) (end 112.381 61.2) (width 0.4) (layer "F.Cu") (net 9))
 (segment (start 109.239999 60.559001) (end 110.49 59.309) (width 0.2) (layer "F.Cu") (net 9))
 (segment (start 136.72 68.58) (end 137.1 68.2) (width 0.4) (layer "F.Cu") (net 9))
 (segment (start 135.19 68.58) (end 136.72 68.58) (width 0.4) (layer "F.Cu") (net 9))
 (segment (start 104.120001 60.559001) (end 109.239999 60.559001) (width 0.2) (layer "F.Cu") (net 9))
 (segment (start 137.1 68.2) (end 137.1 61.8) (width 0.4) (layer "F.Cu") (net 9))
 (segment (start 112.381 61.2) (end 110.49 59.309) (width 0.4) (layer "F.Cu") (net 9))
 (segment (start 137.1 61.8) (end 136.5 61.2) (width 0.4) (layer "F.Cu") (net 9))
 (segment (start 130.1 67.5) (end 125.975 63.375) (width 0.4) (layer "F.Cu") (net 8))
 (segment (start 104.120001 63.099001) (end 109.239999 63.099001) (width 0.2) (layer "F.Cu") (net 8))
 (segment (start 109.239999 63.099001) (end 110.49 61.849) (width 0.2) (layer "F.Cu") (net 8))
 (segment (start 122 63.375) (end 112.016 63.375) (width 0.4) (layer "F.Cu") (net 8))
 (segment (start 102.87 61.849) (end 104.120001 63.099001) (width 0.2) (layer "F.Cu") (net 8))
 (segment (start 112.016 63.375) (end 110.49 61.849) (width 0.4) (layer "F.Cu") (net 8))
 (segment (start 125.975 63.375) (end 122 63.375) (width 0.4) (layer "F.Cu") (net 8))
 (via (at 130.1 67.5) (size 0.8) (drill 0.4) (layers "F.Cu" "B.Cu") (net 8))
 (segment (start 137.6 77.6) (end 135.8 79.4) (width 0.4) (layer "B.Cu") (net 8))
 (segment (start 128.4 69.1) (end 128.4 68.2) (width 0.4) (layer "B.Cu") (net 8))
 (segment (start 129.4 78) (end 129.4 70.1) (width 0.4) (layer "B.Cu") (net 8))
 (segment (start 137.6 73.53) (end 137.6 77.6) (width 0.4) (layer "B.Cu") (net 8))
 (segment (start 135.19 71.12) (end 137.6 73.53) (width 0.4) (layer "B.Cu") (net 8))
 (segment (start 129.1 67.5) (end 130.1 67.5) (width 0.4) (layer "B.Cu") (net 8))
 (segment (start 130.8 79.4) (end 129.4 78) (width 0.4) (layer "B.Cu") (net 8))
 (segment (start 128.4 68.2) (end 129.1 67.5) (width 0.4) (layer "B.Cu") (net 8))
 (segment (start 129.4 70.1) (end 128.4 69.1) (width 0.4) (layer "B.Cu") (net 8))
 (segment (start 135.8 79.4) (end 130.8 79.4) (width 0.4) (layer "B.Cu") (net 8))
 (segment (start 110.726 64.625) (end 110.49 64.389) (width 0.4) (layer "F.Cu") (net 7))
 (segment (start 122 64.625) (end 110.726 64.625) (width 0.4) (layer "F.Cu") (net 7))
 (segment (start 102.87 64.389) (end 104.120001 65.639001) (width 0.2) (layer "F.Cu") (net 7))
 (segment (start 109.239999 65.639001) (end 110.49 64.389) (width 0.2) (layer "F.Cu") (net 7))
 (segment (start 122 64.625) (end 125.425 64.625) (width 0.4) (layer "F.Cu") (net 7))
 (segment (start 125.425 64.625) (end 129.5 68.7) (width 0.4) (layer "F.Cu") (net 7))
 (segment (start 104.120001 65.639001) (end 109.239999 65.639001) (width 0.2) (layer "F.Cu") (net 7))
 (via (at 129.5 68.7) (size 0.8) (drill 0.4) (layers "F.Cu" "B.Cu") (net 7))
 (segment (start 136.8 77.2) (end 135.4 78.6) (width 0.4) (layer "B.Cu") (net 7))
 (segment (start 130.2 77.5) (end 130.2 69.4) (width 0.4) (layer "B.Cu") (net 7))
 (segment (start 135.19 73.66) (end 136.8 75.27) (width 0.4) (layer "B.Cu") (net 7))
 (segment (start 136.8 75.27) (end 136.8 77.2) (width 0.4) (layer "B.Cu") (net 7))
 (segment (start 130.2 69.4) (end 129.5 68.7) (width 0.4) (layer "B.Cu") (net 7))
 (segment (start 131.3 78.6) (end 130.2 77.5) (width 0.4) (layer "B.Cu") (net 7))
 (segment (start 135.4 78.6) (end 131.3 78.6) (width 0.4) (layer "B.Cu") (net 7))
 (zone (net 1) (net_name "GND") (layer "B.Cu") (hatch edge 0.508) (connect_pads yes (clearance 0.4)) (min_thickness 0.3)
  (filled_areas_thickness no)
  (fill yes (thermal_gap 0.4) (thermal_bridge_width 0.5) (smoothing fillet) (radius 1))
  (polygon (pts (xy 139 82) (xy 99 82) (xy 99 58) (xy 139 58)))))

